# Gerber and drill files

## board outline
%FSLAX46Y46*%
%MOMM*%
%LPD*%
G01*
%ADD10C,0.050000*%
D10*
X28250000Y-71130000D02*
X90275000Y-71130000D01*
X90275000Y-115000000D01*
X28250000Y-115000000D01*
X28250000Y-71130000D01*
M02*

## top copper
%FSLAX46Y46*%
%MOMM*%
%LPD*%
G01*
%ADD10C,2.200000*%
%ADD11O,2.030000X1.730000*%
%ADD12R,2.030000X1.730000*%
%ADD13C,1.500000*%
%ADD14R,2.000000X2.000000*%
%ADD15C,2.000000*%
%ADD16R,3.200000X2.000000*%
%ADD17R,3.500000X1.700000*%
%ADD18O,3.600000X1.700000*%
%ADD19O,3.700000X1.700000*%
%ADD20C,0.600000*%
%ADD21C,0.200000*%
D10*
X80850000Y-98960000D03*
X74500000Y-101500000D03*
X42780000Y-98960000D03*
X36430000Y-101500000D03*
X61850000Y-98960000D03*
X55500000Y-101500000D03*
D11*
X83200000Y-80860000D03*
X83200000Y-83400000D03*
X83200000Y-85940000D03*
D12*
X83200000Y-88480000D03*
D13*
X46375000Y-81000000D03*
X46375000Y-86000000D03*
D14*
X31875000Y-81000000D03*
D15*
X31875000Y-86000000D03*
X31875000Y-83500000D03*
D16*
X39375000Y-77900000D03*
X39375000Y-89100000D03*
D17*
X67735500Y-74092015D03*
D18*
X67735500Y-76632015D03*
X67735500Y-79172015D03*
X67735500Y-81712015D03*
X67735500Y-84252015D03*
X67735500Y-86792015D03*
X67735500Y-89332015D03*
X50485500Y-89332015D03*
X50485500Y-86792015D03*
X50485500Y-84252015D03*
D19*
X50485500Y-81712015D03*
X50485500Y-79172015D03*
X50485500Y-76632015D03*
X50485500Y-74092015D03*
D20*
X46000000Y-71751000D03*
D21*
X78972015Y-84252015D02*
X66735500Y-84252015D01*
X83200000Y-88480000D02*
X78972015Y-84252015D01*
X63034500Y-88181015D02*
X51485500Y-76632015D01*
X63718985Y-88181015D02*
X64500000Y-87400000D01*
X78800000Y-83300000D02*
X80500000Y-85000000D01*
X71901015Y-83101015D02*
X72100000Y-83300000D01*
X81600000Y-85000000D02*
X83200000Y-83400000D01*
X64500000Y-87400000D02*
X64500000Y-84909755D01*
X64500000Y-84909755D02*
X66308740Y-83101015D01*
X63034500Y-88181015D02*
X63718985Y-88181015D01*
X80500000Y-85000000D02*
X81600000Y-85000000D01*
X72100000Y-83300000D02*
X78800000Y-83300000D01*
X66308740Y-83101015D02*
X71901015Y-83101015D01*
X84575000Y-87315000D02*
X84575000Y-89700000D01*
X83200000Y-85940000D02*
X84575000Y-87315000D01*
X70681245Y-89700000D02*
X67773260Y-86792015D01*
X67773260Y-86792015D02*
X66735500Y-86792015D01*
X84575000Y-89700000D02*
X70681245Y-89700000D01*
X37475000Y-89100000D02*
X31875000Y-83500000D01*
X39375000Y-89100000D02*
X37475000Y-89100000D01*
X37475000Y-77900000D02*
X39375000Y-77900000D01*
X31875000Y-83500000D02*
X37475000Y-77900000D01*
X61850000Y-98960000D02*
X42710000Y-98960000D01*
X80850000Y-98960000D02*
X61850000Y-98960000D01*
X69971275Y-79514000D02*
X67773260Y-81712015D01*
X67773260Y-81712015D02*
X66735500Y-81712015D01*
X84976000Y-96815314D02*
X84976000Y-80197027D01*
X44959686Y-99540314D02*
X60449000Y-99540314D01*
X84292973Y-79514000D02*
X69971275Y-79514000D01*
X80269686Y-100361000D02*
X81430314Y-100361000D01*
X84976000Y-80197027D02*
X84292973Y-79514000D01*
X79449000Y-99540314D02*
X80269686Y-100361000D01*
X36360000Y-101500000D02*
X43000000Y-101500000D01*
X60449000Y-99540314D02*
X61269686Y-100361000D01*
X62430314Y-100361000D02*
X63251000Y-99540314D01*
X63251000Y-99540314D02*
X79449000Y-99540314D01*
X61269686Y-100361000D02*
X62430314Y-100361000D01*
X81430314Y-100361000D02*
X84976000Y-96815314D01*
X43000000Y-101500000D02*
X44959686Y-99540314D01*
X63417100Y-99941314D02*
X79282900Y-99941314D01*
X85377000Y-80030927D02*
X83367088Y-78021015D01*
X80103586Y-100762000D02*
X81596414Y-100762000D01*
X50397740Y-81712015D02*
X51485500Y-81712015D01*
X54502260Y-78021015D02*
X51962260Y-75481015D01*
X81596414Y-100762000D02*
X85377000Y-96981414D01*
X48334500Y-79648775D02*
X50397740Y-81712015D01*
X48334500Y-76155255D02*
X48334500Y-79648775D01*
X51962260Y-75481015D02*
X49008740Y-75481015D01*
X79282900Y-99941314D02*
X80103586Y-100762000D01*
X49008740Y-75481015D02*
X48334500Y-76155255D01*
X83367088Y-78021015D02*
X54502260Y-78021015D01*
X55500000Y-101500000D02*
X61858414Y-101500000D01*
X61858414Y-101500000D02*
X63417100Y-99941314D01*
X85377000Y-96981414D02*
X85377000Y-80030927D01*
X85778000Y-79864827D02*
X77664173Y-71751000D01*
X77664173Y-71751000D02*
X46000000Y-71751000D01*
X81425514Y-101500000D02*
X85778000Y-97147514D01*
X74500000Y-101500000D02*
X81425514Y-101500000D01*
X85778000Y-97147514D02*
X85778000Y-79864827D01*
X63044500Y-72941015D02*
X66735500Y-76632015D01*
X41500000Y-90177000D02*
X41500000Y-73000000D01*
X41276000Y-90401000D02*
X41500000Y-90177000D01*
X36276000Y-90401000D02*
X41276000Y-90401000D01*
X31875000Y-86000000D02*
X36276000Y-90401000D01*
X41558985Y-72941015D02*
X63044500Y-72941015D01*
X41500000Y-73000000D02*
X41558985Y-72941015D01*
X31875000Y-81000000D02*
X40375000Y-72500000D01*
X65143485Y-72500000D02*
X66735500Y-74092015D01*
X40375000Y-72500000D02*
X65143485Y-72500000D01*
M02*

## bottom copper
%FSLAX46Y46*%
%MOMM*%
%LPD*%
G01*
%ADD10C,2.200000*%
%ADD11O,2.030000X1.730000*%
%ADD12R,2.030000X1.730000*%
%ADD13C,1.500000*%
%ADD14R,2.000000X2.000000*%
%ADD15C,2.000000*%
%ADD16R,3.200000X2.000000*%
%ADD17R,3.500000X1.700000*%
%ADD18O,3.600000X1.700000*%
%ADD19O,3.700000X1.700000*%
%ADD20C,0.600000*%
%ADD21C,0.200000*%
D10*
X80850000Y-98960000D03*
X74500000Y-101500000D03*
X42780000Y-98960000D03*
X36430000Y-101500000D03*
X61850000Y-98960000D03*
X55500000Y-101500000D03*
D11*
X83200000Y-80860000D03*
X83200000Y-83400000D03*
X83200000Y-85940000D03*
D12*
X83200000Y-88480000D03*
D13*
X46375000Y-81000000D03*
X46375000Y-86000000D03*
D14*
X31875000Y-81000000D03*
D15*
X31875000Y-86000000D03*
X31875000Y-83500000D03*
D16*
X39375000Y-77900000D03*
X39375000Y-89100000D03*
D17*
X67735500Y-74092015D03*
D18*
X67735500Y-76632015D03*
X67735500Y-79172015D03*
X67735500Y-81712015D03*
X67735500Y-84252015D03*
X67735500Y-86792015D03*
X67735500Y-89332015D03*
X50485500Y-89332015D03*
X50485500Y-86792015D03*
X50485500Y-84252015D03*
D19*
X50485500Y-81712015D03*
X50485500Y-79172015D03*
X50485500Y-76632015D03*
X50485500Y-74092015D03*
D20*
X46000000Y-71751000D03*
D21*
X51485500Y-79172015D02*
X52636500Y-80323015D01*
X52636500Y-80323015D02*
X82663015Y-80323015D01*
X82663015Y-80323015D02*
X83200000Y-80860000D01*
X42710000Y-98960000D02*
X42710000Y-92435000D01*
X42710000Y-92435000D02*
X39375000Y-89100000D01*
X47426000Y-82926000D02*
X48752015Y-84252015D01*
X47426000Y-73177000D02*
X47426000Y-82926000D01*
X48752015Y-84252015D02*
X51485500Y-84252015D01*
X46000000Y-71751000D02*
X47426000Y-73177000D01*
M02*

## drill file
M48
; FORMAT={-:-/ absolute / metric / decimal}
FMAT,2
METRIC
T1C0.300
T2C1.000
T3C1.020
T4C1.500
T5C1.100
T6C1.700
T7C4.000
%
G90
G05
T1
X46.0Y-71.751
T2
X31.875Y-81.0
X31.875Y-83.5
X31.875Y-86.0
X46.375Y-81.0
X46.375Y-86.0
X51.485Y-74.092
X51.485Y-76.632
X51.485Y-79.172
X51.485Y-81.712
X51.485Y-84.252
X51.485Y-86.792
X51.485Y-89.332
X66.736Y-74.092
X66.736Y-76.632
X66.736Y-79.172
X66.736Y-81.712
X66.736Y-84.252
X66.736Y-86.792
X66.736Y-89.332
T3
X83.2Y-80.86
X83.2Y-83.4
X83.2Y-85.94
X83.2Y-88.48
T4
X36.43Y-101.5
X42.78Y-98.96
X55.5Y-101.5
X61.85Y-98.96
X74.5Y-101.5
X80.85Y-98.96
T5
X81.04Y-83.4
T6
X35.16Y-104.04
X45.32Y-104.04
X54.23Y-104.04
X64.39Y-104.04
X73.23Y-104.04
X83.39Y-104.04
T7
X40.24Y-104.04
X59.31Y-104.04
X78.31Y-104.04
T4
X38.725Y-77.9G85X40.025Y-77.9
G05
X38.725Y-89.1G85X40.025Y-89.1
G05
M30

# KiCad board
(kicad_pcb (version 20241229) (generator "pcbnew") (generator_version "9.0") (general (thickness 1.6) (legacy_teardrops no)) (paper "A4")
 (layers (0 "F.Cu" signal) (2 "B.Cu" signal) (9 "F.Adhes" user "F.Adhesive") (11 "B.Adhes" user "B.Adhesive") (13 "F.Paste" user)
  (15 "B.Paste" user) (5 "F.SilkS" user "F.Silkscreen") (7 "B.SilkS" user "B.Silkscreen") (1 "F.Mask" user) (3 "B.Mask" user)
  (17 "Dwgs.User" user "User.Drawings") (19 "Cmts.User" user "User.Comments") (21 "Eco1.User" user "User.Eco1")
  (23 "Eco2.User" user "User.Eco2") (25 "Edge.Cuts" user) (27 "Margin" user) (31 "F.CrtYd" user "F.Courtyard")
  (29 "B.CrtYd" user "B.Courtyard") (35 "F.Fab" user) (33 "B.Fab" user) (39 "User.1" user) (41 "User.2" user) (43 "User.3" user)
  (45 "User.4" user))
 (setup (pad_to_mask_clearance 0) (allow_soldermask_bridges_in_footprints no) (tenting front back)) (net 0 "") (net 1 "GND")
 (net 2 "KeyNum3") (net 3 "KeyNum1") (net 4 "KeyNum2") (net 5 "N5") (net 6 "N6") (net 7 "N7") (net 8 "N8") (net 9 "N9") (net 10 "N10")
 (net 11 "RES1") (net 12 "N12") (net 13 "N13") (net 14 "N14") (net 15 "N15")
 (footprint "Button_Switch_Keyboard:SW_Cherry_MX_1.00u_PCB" (layer "F.Cu") (at 80.85 98.96)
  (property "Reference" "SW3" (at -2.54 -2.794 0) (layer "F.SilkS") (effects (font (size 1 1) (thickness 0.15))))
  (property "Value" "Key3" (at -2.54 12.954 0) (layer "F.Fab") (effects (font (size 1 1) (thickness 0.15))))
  (pad "" np_thru_hole circle (at -7.62 5.08) (size 1.7 1.7) (drill 1.7) (layers "*.Cu" "*.Mask"))
  (pad "" np_thru_hole circle (at -2.54 5.08) (size 4 4) (drill 4) (layers "*.Cu" "*.Mask"))
  (pad "" np_thru_hole circle (at 2.54 5.08) (size 1.7 1.7) (drill 1.7) (layers "*.Cu" "*.Mask"))
  (pad "1" thru_hole circle (at 0 0) (size 2.2 2.2) (drill 1.5) (layers "*.Cu" "*.Mask") (remove_unused_layers no) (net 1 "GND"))
  (pad "2" thru_hole circle (at -6.35 2.54) (size 2.2 2.2) (drill 1.5) (layers "*.Cu" "*.Mask") (remove_unused_layers no) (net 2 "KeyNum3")))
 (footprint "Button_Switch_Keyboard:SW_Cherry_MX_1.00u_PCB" (layer "F.Cu") (at 42.78 98.96)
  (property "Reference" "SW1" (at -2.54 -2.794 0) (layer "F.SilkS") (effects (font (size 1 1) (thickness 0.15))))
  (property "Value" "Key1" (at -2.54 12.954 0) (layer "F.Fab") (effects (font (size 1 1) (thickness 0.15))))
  (pad "" np_thru_hole circle (at -7.62 5.08) (size 1.7 1.7) (drill 1.7) (layers "*.Cu" "*.Mask"))
  (pad "" np_thru_hole circle (at -2.54 5.08) (size 4 4) (drill 4) (layers "*.Cu" "*.Mask"))
  (pad "" np_thru_hole circle (at 2.54 5.08) (size 1.7 1.7) (drill 1.7) (layers "*.Cu" "*.Mask"))
  (pad "1" thru_hole circle (at 0 0) (size 2.2 2.2) (drill 1.5) (layers "*.Cu" "*.Mask") (remove_unused_layers no) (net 1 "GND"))
  (pad "2" thru_hole circle (at -6.35 2.54) (size 2.2 2.2) (drill 1.5) (layers "*.Cu" "*.Mask") (remove_unused_layers no) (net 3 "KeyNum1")))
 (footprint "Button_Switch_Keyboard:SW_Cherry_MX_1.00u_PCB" (layer "F.Cu") (at 61.85 98.96)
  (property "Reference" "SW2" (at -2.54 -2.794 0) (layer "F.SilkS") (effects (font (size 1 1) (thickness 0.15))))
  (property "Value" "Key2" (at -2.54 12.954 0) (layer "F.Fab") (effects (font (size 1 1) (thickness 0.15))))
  (pad "" np_thru_hole circle (at -7.62 5.08) (size 1.7 1.7) (drill 1.7) (layers "*.Cu" "*.Mask"))
  (pad "" np_thru_hole circle (at -2.54 5.08) (size 4 4) (drill 4) (layers "*.Cu" "*.Mask"))
  (pad "" np_thru_hole circle (at 2.54 5.08) (size 1.7 1.7) (drill 1.7) (layers "*.Cu" "*.Mask"))
  (pad "1" thru_hole circle (at 0 0) (size 2.2 2.2) (drill 1.5) (layers "*.Cu" "*.Mask") (remove_unused_layers no) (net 1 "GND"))
  (pad "2" thru_hole circle (at -6.35 2.54) (size 2.2 2.2) (drill 1.5) (layers "*.Cu" "*.Mask") (remove_unused_layers no) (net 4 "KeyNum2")))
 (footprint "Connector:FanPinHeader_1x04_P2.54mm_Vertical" (layer "F.Cu") (at 83.2 88.48 90)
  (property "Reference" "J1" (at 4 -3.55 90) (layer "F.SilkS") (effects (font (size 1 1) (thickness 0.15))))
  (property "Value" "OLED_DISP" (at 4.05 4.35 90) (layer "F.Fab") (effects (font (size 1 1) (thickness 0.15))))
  (pad "" np_thru_hole circle (at 5.08 -2.16 180) (size 1.1 1.1) (drill 1.1) (layers "*.Cu" "*.Mask"))
  (pad "1" thru_hole oval (at 7.62 0 180) (size 2.03 1.73) (drill 1.02) (layers "*.Cu" "*.Mask") (remove_unused_layers no) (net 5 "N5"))
  (pad "2" thru_hole oval (at 5.08 0 180) (size 2.03 1.73) (drill 1.02) (layers "*.Cu" "*.Mask") (remove_unused_layers no) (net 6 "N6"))
  (pad "3" thru_hole oval (at 2.54 0 180) (size 2.03 1.73) (drill 1.02) (layers "*.Cu" "*.Mask") (remove_unused_layers no) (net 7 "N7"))
  (pad "4" thru_hole rect (at 0 0 180) (size 2.03 1.73) (drill 1.02) (layers "*.Cu" "*.Mask") (remove_unused_layers no) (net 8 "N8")))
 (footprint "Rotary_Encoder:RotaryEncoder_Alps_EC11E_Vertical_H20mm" (layer "F.Cu") (at 31.875 81)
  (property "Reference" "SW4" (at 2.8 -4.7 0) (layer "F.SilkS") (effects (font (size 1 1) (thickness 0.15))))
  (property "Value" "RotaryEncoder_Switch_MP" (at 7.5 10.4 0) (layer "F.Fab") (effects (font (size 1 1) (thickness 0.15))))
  (pad "" thru_hole circle (at 14.5 0) (size 1.5 1.5) (drill 1) (layers "*.Cu" "*.Mask") (remove_unused_layers no))
  (pad "" thru_hole circle (at 14.5 5) (size 1.5 1.5) (drill 1) (layers "*.Cu" "*.Mask") (remove_unused_layers no))
  (pad "A" thru_hole rect (at 0 0) (size 2 2) (drill 1) (layers "*.Cu" "*.Mask") (remove_unused_layers no) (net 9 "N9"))
  (pad "B" thru_hole circle (at 0 5) (size 2 2) (drill 1) (layers "*.Cu" "*.Mask") (remove_unused_layers no) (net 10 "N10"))
  (pad "C" thru_hole circle (at 0 2.5) (size 2 2) (drill 1) (layers "*.Cu" "*.Mask") (remove_unused_layers no) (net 1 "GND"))
  (pad "MP" thru_hole rect (at 7.5 -3.1) (size 3.2 2) (drill oval 2.8 1.5) (layers "*.Cu" "*.Mask") (remove_unused_layers no) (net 1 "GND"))
  (pad "MP" thru_hole rect (at 7.5 8.1) (size 3.2 2) (drill oval 2.8 1.5) (layers "*.Cu" "*.Mask") (remove_unused_layers no) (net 1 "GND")))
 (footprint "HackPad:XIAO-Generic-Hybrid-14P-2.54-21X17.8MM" (layer "B.Cu") (at 59.1105 81.712015 180)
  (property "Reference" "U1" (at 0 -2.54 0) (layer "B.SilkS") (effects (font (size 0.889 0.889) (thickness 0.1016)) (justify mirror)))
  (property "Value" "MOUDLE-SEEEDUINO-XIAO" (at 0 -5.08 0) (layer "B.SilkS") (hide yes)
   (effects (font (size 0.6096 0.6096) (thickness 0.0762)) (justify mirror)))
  (pad "1" thru_hole rect (at -7.625 7.62 180) (size 3.5 1.7) (drill 1 (offset -1 0)) (layers "*.Cu" "*.Mask") (remove_unused_layers no)
   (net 9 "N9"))
  (pad "2" thru_hole oval (at -7.625 5.08 180) (size 3.6 1.7) (drill 1 (offset -1 0)) (layers "*.Cu" "*.Mask") (remove_unused_layers no)
   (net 10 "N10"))
  (pad "3" thru_hole oval (at -7.625 2.54 180) (size 3.6 1.7) (drill 1 (offset -1 0)) (layers "*.Cu" "*.Mask") (remove_unused_layers no)
   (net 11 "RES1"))
  (pad "4" thru_hole oval (at -7.625 0 180) (size 3.6 1.7) (drill 1 (offset -1 0)) (layers "*.Cu" "*.Mask") (remove_unused_layers no)
   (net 3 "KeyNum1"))
  (pad "5" thru_hole oval (at -7.625 -2.54 180) (size 3.6 1.7) (drill 1 (offset -1 0)) (layers "*.Cu" "*.Mask") (remove_unused_layers no)
   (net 8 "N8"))
  (pad "6" thru_hole oval (at -7.625 -5.08) (size 3.6 1.7) (drill 1 (offset 1 0)) (layers "*.Cu" "*.Mask") (remove_unused_layers no)
   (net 7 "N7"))
  (pad "7" thru_hole oval (at -7.625 -7.62 180) (size 3.6 1.7) (drill 1 (offset -1 0)) (layers "*.Cu" "*.Mask") (remove_unused_layers no)
   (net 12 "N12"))
  (pad "8" thru_hole oval (at 7.625 -7.62 180) (size 3.6 1.7) (drill 1 (offset 1 0)) (layers "*.Cu" "*.Mask") (remove_unused_layers no)
   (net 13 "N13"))
  (pad "9" thru_hole oval (at 7.625 -5.08 180) (size 3.6 1.7) (drill 1 (offset 1 0)) (layers "*.Cu" "*.Mask") (remove_unused_layers no)
   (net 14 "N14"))
  (pad "10" thru_hole oval (at 7.625 -2.54 180) (size 3.6 1.7) (drill 1 (offset 1 0)) (layers "*.Cu" "*.Mask") (remove_unused_layers no)
   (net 2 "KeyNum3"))
  (pad "11" thru_hole oval (at 7.625 0 180) (size 3.7 1.7) (drill 1 (offset 1 0)) (layers "*.Cu" "*.Mask") (remove_unused_layers no)
   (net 4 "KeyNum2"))
  (pad "12" thru_hole oval (at 7.625 2.54 180) (size 3.7 1.7) (drill 1 (offset 1 0)) (layers "*.Cu" "*.Mask") (remove_unused_layers no)
   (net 5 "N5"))
  (pad "13" thru_hole oval (at 7.625 5.08 180) (size 3.7 1.7) (drill 1 (offset 1 0)) (layers "*.Cu" "*.Mask") (remove_unused_layers no)
   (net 6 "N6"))
  (pad "14" thru_hole oval (at 7.625 7.62 180) (size 3.7 1.7) (drill 1 (offset 1 0)) (layers "*.Cu" "*.Mask") (remove_unused_layers no)
   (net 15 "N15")))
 (gr_rect (start 28.25 71.13) (end 90.275 115) (stroke (width 0.05) (type default)) (fill no) (layer "Edge.Cuts"))
 (segment (start 78.972015 84.252015) (end 66.7355 84.252015) (width 0.2) (layer "F.Cu") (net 8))
 (segment (start 83.2 88.48) (end 78.972015 84.252015) (width 0.2) (layer "F.Cu") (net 8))
 (segment (start 63.0345 88.181015) (end 51.4855 76.632015) (width 0.2) (layer "F.Cu") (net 6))
 (segment (start 63.718985 88.181015) (end 64.5 87.4) (width 0.2) (layer "F.Cu") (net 6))
 (segment (start 78.8 83.3) (end 80.5 85) (width 0.2) (layer "F.Cu") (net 6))
 (segment (start 71.901015 83.101015) (end 72.1 83.3) (width 0.2) (layer "F.Cu") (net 6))
 (segment (start 81.6 85) (end 83.2 83.4) (width 0.2) (layer "F.Cu") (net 6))
 (segment (start 64.5 87.4) (end 64.5 84.909755) (width 0.2) (layer "F.Cu") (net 6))
 (segment (start 64.5 84.909755) (end 66.30874 83.101015) (width 0.2) (layer "F.Cu") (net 6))
 (segment (start 63.0345 88.181015) (end 63.718985 88.181015) (width 0.2) (layer "F.Cu") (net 6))
 (segment (start 80.5 85) (end 81.6 85) (width 0.2) (layer "F.Cu") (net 6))
 (segment (start 72.1 83.3) (end 78.8 83.3) (width 0.2) (layer "F.Cu") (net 6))
 (segment (start 66.30874 83.101015) (end 71.901015 83.101015) (width 0.2) (layer "F.Cu") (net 6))
 (segment (start 51.4855 79.172015) (end 52.6365 80.323015) (width 0.2) (layer "B.Cu") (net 5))
 (segment (start 52.6365 80.323015) (end 82.663015 80.323015) (width 0.2) (layer "B.Cu") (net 5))
 (segment (start 82.663015 80.323015) (end 83.2 80.86) (width 0.2) (layer "B.Cu") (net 5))
 (segment (start 84.575 87.315) (end 84.575 89.7) (width 0.2) (layer "F.Cu") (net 7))
 (segment (start 83.2 85.94) (end 84.575 87.315) (width 0.2) (layer "F.Cu") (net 7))
 (segment (start 70.681245 89.7) (end 67.77326 86.792015) (width 0.2) (layer "F.Cu") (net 7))
 (segment (start 67.77326 86.792015) (end 66.7355 86.792015) (width 0.2) (layer "F.Cu") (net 7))
 (segment (start 84.575 89.7) (end 70.681245 89.7) (width 0.2) (layer "F.Cu") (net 7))
 (segment (start 37.475 89.1) (end 31.875 83.5) (width 0.2) (layer "F.Cu") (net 1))
 (segment (start 39.375 89.1) (end 37.475 89.1) (width 0.2) (layer "F.Cu") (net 1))
 (segment (start 37.475 77.9) (end 39.375 77.9) (width 0.2) (layer "F.Cu") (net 1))
 (segment (start 31.875 83.5) (end 37.475 77.9) (width 0.2) (layer "F.Cu") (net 1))
 (segment (start 61.85 98.96) (end 42.71 98.96) (width 0.2) (layer "F.Cu") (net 1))
 (segment (start 80.85 98.96) (end 61.85 98.96) (width 0.2) (layer "F.Cu") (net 1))
 (segment (start 42.71 98.96) (end 42.71 92.435) (width 0.2) (layer "B.Cu") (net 1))
 (segment (start 42.71 92.435) (end 39.375 89.1) (width 0.2) (layer "B.Cu") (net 1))
 (segment (start 69.971275 79.514) (end 67.77326 81.712015) (width 0.2) (layer "F.Cu") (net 3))
 (segment (start 67.77326 81.712015) (end 66.7355 81.712015) (width 0.2) (layer "F.Cu") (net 3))
 (segment (start 84.976 96.815314) (end 84.976 80.197027) (width 0.2) (layer "F.Cu") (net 3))
 (segment (start 44.959686 99.540314) (end 60.449 99.540314) (width 0.2) (layer "F.Cu") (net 3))
 (segment (start 84.292973 79.514) (end 69.971275 79.514) (width 0.2) (layer "F.Cu") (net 3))
 (segment (start 80.269686 100.361) (end 81.430314 100.361) (width 0.2) (layer "F.Cu") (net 3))
 (segment (start 84.976 80.197027) (end 84.292973 79.514) (width 0.2) (layer "F.Cu") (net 3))
 (segment (start 79.449 99.540314) (end 80.269686 100.361) (width 0.2) (layer "F.Cu") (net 3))
 (segment (start 36.36 101.5) (end 43 101.5) (width 0.2) (layer "F.Cu") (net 3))
 (segment (start 60.449 99.540314) (end 61.269686 100.361) (width 0.2) (layer "F.Cu") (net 3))
 (segment (start 62.430314 100.361) (end 63.251 99.540314) (width 0.2) (layer "F.Cu") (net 3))
 (segment (start 63.251 99.540314) (end 79.449 99.540314) (width 0.2) (layer "F.Cu") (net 3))
 (segment (start 61.269686 100.361) (end 62.430314 100.361) (width 0.2) (layer "F.Cu") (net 3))
 (segment (start 81.430314 100.361) (end 84.976 96.815314) (width 0.2) (layer "F.Cu") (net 3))
 (segment (start 43 101.5) (end 44.959686 99.540314) (width 0.2) (layer "F.Cu") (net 3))
 (segment (start 63.4171 99.941314) (end 79.2829 99.941314) (width 0.2) (layer "F.Cu") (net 4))
 (segment (start 85.377 80.030927) (end 83.367088 78.021015) (width 0.2) (layer "F.Cu") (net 4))
 (segment (start 80.103586 100.762) (end 81.596414 100.762) (width 0.2) (layer "F.Cu") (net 4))
 (segment (start 50.39774 81.712015) (end 51.4855 81.712015) (width 0.2) (layer "F.Cu") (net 4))
 (segment (start 54.50226 78.021015) (end 51.96226 75.481015) (width 0.2) (layer "F.Cu") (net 4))
 (segment (start 81.596414 100.762) (end 85.377 96.981414) (width 0.2) (layer "F.Cu") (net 4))
 (segment (start 48.3345 79.648775) (end 50.39774 81.712015) (width 0.2) (layer "F.Cu") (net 4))
 (segment (start 48.3345 76.155255) (end 48.3345 79.648775) (width 0.2) (layer "F.Cu") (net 4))
 (segment (start 51.96226 75.481015) (end 49.00874 75.481015) (width 0.2) (layer "F.Cu") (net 4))
 (segment (start 79.2829 99.941314) (end 80.103586 100.762) (width 0.2) (layer "F.Cu") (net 4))
 (segment (start 49.00874 75.481015) (end 48.3345 76.155255) (width 0.2) (layer "F.Cu") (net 4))
 (segment (start 83.367088 78.021015) (end 54.50226 78.021015) (width 0.2) (layer "F.Cu") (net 4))
 (segment (start 55.5 101.5) (end 61.858414 101.5) (width 0.2) (layer "F.Cu") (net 4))
 (segment (start 61.858414 101.5) (end 63.4171 99.941314) (width 0.2) (layer "F.Cu") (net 4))
 (segment (start 85.377 96.981414) (end 85.377 80.030927) (width 0.2) (layer "F.Cu") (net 4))
 (segment (start 85.778 79.864827) (end 77.664173 71.751) (width 0.2) (layer "F.Cu") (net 2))
 (segment (start 77.664173 71.751) (end 46 71.751) (width 0.2) (layer "F.Cu") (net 2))
 (segment (start 81.425514 101.5) (end 85.778 97.147514) (width 0.2) (layer "F.Cu") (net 2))
 (segment (start 74.5 101.5) (end 81.425514 101.5) (width 0.2) (layer "F.Cu") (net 2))
 (segment (start 85.778 97.147514) (end 85.778 79.864827) (width 0.2) (layer "F.Cu") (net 2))
 (via (at 46 71.751) (size 0.6) (drill 0.3) (layers "F.Cu" "B.Cu") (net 2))
 (segment (start 47.426 82.926) (end 48.752015 84.252015) (width 0.2) (layer "B.Cu") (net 2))
 (segment (start 47.426 73.177) (end 47.426 82.926) (width 0.2) (layer "B.Cu") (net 2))
 (segment (start 48.752015 84.252015) (end 51.4855 84.252015) (width 0.2) (layer "B.Cu") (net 2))
 (segment (start 46 71.751) (end 47.426 73.177) (width 0.2) (layer "B.Cu") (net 2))
 (segment (start 63.0445 72.941015) (end 66.7355 76.632015) (width 0.2) (layer "F.Cu") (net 10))
 (segment (start 41.5 90.177) (end 41.5 73) (width 0.2) (layer "F.Cu") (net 10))
 (segment (start 41.276 90.401) (end 41.5 90.177) (width 0.2) (layer "F.Cu") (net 10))
 (segment (start 36.276 90.401) (end 41.276 90.401) (width 0.2) (layer "F.Cu") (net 10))
 (segment (start 31.875 86) (end 36.276 90.401) (width 0.2) (layer "F.Cu") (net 10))
 (segment (start 41.558985 72.941015) (end 63.0445 72.941015) (width 0.2) (layer "F.Cu") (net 10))
 (segment (start 41.5 73) (end 41.558985 72.941015) (width 0.2) (layer "F.Cu") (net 10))
 (segment (start 31.875 81) (end 40.375 72.5) (width 0.2) (layer "F.Cu") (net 9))
 (segment (start 65.143485 72.5) (end 66.7355 74.092015) (width 0.2) (layer "F.Cu") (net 9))
 (segment (start 40.375 72.5) (end 65.143485 72.5) (width 0.2) (layer "F.Cu") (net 9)))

